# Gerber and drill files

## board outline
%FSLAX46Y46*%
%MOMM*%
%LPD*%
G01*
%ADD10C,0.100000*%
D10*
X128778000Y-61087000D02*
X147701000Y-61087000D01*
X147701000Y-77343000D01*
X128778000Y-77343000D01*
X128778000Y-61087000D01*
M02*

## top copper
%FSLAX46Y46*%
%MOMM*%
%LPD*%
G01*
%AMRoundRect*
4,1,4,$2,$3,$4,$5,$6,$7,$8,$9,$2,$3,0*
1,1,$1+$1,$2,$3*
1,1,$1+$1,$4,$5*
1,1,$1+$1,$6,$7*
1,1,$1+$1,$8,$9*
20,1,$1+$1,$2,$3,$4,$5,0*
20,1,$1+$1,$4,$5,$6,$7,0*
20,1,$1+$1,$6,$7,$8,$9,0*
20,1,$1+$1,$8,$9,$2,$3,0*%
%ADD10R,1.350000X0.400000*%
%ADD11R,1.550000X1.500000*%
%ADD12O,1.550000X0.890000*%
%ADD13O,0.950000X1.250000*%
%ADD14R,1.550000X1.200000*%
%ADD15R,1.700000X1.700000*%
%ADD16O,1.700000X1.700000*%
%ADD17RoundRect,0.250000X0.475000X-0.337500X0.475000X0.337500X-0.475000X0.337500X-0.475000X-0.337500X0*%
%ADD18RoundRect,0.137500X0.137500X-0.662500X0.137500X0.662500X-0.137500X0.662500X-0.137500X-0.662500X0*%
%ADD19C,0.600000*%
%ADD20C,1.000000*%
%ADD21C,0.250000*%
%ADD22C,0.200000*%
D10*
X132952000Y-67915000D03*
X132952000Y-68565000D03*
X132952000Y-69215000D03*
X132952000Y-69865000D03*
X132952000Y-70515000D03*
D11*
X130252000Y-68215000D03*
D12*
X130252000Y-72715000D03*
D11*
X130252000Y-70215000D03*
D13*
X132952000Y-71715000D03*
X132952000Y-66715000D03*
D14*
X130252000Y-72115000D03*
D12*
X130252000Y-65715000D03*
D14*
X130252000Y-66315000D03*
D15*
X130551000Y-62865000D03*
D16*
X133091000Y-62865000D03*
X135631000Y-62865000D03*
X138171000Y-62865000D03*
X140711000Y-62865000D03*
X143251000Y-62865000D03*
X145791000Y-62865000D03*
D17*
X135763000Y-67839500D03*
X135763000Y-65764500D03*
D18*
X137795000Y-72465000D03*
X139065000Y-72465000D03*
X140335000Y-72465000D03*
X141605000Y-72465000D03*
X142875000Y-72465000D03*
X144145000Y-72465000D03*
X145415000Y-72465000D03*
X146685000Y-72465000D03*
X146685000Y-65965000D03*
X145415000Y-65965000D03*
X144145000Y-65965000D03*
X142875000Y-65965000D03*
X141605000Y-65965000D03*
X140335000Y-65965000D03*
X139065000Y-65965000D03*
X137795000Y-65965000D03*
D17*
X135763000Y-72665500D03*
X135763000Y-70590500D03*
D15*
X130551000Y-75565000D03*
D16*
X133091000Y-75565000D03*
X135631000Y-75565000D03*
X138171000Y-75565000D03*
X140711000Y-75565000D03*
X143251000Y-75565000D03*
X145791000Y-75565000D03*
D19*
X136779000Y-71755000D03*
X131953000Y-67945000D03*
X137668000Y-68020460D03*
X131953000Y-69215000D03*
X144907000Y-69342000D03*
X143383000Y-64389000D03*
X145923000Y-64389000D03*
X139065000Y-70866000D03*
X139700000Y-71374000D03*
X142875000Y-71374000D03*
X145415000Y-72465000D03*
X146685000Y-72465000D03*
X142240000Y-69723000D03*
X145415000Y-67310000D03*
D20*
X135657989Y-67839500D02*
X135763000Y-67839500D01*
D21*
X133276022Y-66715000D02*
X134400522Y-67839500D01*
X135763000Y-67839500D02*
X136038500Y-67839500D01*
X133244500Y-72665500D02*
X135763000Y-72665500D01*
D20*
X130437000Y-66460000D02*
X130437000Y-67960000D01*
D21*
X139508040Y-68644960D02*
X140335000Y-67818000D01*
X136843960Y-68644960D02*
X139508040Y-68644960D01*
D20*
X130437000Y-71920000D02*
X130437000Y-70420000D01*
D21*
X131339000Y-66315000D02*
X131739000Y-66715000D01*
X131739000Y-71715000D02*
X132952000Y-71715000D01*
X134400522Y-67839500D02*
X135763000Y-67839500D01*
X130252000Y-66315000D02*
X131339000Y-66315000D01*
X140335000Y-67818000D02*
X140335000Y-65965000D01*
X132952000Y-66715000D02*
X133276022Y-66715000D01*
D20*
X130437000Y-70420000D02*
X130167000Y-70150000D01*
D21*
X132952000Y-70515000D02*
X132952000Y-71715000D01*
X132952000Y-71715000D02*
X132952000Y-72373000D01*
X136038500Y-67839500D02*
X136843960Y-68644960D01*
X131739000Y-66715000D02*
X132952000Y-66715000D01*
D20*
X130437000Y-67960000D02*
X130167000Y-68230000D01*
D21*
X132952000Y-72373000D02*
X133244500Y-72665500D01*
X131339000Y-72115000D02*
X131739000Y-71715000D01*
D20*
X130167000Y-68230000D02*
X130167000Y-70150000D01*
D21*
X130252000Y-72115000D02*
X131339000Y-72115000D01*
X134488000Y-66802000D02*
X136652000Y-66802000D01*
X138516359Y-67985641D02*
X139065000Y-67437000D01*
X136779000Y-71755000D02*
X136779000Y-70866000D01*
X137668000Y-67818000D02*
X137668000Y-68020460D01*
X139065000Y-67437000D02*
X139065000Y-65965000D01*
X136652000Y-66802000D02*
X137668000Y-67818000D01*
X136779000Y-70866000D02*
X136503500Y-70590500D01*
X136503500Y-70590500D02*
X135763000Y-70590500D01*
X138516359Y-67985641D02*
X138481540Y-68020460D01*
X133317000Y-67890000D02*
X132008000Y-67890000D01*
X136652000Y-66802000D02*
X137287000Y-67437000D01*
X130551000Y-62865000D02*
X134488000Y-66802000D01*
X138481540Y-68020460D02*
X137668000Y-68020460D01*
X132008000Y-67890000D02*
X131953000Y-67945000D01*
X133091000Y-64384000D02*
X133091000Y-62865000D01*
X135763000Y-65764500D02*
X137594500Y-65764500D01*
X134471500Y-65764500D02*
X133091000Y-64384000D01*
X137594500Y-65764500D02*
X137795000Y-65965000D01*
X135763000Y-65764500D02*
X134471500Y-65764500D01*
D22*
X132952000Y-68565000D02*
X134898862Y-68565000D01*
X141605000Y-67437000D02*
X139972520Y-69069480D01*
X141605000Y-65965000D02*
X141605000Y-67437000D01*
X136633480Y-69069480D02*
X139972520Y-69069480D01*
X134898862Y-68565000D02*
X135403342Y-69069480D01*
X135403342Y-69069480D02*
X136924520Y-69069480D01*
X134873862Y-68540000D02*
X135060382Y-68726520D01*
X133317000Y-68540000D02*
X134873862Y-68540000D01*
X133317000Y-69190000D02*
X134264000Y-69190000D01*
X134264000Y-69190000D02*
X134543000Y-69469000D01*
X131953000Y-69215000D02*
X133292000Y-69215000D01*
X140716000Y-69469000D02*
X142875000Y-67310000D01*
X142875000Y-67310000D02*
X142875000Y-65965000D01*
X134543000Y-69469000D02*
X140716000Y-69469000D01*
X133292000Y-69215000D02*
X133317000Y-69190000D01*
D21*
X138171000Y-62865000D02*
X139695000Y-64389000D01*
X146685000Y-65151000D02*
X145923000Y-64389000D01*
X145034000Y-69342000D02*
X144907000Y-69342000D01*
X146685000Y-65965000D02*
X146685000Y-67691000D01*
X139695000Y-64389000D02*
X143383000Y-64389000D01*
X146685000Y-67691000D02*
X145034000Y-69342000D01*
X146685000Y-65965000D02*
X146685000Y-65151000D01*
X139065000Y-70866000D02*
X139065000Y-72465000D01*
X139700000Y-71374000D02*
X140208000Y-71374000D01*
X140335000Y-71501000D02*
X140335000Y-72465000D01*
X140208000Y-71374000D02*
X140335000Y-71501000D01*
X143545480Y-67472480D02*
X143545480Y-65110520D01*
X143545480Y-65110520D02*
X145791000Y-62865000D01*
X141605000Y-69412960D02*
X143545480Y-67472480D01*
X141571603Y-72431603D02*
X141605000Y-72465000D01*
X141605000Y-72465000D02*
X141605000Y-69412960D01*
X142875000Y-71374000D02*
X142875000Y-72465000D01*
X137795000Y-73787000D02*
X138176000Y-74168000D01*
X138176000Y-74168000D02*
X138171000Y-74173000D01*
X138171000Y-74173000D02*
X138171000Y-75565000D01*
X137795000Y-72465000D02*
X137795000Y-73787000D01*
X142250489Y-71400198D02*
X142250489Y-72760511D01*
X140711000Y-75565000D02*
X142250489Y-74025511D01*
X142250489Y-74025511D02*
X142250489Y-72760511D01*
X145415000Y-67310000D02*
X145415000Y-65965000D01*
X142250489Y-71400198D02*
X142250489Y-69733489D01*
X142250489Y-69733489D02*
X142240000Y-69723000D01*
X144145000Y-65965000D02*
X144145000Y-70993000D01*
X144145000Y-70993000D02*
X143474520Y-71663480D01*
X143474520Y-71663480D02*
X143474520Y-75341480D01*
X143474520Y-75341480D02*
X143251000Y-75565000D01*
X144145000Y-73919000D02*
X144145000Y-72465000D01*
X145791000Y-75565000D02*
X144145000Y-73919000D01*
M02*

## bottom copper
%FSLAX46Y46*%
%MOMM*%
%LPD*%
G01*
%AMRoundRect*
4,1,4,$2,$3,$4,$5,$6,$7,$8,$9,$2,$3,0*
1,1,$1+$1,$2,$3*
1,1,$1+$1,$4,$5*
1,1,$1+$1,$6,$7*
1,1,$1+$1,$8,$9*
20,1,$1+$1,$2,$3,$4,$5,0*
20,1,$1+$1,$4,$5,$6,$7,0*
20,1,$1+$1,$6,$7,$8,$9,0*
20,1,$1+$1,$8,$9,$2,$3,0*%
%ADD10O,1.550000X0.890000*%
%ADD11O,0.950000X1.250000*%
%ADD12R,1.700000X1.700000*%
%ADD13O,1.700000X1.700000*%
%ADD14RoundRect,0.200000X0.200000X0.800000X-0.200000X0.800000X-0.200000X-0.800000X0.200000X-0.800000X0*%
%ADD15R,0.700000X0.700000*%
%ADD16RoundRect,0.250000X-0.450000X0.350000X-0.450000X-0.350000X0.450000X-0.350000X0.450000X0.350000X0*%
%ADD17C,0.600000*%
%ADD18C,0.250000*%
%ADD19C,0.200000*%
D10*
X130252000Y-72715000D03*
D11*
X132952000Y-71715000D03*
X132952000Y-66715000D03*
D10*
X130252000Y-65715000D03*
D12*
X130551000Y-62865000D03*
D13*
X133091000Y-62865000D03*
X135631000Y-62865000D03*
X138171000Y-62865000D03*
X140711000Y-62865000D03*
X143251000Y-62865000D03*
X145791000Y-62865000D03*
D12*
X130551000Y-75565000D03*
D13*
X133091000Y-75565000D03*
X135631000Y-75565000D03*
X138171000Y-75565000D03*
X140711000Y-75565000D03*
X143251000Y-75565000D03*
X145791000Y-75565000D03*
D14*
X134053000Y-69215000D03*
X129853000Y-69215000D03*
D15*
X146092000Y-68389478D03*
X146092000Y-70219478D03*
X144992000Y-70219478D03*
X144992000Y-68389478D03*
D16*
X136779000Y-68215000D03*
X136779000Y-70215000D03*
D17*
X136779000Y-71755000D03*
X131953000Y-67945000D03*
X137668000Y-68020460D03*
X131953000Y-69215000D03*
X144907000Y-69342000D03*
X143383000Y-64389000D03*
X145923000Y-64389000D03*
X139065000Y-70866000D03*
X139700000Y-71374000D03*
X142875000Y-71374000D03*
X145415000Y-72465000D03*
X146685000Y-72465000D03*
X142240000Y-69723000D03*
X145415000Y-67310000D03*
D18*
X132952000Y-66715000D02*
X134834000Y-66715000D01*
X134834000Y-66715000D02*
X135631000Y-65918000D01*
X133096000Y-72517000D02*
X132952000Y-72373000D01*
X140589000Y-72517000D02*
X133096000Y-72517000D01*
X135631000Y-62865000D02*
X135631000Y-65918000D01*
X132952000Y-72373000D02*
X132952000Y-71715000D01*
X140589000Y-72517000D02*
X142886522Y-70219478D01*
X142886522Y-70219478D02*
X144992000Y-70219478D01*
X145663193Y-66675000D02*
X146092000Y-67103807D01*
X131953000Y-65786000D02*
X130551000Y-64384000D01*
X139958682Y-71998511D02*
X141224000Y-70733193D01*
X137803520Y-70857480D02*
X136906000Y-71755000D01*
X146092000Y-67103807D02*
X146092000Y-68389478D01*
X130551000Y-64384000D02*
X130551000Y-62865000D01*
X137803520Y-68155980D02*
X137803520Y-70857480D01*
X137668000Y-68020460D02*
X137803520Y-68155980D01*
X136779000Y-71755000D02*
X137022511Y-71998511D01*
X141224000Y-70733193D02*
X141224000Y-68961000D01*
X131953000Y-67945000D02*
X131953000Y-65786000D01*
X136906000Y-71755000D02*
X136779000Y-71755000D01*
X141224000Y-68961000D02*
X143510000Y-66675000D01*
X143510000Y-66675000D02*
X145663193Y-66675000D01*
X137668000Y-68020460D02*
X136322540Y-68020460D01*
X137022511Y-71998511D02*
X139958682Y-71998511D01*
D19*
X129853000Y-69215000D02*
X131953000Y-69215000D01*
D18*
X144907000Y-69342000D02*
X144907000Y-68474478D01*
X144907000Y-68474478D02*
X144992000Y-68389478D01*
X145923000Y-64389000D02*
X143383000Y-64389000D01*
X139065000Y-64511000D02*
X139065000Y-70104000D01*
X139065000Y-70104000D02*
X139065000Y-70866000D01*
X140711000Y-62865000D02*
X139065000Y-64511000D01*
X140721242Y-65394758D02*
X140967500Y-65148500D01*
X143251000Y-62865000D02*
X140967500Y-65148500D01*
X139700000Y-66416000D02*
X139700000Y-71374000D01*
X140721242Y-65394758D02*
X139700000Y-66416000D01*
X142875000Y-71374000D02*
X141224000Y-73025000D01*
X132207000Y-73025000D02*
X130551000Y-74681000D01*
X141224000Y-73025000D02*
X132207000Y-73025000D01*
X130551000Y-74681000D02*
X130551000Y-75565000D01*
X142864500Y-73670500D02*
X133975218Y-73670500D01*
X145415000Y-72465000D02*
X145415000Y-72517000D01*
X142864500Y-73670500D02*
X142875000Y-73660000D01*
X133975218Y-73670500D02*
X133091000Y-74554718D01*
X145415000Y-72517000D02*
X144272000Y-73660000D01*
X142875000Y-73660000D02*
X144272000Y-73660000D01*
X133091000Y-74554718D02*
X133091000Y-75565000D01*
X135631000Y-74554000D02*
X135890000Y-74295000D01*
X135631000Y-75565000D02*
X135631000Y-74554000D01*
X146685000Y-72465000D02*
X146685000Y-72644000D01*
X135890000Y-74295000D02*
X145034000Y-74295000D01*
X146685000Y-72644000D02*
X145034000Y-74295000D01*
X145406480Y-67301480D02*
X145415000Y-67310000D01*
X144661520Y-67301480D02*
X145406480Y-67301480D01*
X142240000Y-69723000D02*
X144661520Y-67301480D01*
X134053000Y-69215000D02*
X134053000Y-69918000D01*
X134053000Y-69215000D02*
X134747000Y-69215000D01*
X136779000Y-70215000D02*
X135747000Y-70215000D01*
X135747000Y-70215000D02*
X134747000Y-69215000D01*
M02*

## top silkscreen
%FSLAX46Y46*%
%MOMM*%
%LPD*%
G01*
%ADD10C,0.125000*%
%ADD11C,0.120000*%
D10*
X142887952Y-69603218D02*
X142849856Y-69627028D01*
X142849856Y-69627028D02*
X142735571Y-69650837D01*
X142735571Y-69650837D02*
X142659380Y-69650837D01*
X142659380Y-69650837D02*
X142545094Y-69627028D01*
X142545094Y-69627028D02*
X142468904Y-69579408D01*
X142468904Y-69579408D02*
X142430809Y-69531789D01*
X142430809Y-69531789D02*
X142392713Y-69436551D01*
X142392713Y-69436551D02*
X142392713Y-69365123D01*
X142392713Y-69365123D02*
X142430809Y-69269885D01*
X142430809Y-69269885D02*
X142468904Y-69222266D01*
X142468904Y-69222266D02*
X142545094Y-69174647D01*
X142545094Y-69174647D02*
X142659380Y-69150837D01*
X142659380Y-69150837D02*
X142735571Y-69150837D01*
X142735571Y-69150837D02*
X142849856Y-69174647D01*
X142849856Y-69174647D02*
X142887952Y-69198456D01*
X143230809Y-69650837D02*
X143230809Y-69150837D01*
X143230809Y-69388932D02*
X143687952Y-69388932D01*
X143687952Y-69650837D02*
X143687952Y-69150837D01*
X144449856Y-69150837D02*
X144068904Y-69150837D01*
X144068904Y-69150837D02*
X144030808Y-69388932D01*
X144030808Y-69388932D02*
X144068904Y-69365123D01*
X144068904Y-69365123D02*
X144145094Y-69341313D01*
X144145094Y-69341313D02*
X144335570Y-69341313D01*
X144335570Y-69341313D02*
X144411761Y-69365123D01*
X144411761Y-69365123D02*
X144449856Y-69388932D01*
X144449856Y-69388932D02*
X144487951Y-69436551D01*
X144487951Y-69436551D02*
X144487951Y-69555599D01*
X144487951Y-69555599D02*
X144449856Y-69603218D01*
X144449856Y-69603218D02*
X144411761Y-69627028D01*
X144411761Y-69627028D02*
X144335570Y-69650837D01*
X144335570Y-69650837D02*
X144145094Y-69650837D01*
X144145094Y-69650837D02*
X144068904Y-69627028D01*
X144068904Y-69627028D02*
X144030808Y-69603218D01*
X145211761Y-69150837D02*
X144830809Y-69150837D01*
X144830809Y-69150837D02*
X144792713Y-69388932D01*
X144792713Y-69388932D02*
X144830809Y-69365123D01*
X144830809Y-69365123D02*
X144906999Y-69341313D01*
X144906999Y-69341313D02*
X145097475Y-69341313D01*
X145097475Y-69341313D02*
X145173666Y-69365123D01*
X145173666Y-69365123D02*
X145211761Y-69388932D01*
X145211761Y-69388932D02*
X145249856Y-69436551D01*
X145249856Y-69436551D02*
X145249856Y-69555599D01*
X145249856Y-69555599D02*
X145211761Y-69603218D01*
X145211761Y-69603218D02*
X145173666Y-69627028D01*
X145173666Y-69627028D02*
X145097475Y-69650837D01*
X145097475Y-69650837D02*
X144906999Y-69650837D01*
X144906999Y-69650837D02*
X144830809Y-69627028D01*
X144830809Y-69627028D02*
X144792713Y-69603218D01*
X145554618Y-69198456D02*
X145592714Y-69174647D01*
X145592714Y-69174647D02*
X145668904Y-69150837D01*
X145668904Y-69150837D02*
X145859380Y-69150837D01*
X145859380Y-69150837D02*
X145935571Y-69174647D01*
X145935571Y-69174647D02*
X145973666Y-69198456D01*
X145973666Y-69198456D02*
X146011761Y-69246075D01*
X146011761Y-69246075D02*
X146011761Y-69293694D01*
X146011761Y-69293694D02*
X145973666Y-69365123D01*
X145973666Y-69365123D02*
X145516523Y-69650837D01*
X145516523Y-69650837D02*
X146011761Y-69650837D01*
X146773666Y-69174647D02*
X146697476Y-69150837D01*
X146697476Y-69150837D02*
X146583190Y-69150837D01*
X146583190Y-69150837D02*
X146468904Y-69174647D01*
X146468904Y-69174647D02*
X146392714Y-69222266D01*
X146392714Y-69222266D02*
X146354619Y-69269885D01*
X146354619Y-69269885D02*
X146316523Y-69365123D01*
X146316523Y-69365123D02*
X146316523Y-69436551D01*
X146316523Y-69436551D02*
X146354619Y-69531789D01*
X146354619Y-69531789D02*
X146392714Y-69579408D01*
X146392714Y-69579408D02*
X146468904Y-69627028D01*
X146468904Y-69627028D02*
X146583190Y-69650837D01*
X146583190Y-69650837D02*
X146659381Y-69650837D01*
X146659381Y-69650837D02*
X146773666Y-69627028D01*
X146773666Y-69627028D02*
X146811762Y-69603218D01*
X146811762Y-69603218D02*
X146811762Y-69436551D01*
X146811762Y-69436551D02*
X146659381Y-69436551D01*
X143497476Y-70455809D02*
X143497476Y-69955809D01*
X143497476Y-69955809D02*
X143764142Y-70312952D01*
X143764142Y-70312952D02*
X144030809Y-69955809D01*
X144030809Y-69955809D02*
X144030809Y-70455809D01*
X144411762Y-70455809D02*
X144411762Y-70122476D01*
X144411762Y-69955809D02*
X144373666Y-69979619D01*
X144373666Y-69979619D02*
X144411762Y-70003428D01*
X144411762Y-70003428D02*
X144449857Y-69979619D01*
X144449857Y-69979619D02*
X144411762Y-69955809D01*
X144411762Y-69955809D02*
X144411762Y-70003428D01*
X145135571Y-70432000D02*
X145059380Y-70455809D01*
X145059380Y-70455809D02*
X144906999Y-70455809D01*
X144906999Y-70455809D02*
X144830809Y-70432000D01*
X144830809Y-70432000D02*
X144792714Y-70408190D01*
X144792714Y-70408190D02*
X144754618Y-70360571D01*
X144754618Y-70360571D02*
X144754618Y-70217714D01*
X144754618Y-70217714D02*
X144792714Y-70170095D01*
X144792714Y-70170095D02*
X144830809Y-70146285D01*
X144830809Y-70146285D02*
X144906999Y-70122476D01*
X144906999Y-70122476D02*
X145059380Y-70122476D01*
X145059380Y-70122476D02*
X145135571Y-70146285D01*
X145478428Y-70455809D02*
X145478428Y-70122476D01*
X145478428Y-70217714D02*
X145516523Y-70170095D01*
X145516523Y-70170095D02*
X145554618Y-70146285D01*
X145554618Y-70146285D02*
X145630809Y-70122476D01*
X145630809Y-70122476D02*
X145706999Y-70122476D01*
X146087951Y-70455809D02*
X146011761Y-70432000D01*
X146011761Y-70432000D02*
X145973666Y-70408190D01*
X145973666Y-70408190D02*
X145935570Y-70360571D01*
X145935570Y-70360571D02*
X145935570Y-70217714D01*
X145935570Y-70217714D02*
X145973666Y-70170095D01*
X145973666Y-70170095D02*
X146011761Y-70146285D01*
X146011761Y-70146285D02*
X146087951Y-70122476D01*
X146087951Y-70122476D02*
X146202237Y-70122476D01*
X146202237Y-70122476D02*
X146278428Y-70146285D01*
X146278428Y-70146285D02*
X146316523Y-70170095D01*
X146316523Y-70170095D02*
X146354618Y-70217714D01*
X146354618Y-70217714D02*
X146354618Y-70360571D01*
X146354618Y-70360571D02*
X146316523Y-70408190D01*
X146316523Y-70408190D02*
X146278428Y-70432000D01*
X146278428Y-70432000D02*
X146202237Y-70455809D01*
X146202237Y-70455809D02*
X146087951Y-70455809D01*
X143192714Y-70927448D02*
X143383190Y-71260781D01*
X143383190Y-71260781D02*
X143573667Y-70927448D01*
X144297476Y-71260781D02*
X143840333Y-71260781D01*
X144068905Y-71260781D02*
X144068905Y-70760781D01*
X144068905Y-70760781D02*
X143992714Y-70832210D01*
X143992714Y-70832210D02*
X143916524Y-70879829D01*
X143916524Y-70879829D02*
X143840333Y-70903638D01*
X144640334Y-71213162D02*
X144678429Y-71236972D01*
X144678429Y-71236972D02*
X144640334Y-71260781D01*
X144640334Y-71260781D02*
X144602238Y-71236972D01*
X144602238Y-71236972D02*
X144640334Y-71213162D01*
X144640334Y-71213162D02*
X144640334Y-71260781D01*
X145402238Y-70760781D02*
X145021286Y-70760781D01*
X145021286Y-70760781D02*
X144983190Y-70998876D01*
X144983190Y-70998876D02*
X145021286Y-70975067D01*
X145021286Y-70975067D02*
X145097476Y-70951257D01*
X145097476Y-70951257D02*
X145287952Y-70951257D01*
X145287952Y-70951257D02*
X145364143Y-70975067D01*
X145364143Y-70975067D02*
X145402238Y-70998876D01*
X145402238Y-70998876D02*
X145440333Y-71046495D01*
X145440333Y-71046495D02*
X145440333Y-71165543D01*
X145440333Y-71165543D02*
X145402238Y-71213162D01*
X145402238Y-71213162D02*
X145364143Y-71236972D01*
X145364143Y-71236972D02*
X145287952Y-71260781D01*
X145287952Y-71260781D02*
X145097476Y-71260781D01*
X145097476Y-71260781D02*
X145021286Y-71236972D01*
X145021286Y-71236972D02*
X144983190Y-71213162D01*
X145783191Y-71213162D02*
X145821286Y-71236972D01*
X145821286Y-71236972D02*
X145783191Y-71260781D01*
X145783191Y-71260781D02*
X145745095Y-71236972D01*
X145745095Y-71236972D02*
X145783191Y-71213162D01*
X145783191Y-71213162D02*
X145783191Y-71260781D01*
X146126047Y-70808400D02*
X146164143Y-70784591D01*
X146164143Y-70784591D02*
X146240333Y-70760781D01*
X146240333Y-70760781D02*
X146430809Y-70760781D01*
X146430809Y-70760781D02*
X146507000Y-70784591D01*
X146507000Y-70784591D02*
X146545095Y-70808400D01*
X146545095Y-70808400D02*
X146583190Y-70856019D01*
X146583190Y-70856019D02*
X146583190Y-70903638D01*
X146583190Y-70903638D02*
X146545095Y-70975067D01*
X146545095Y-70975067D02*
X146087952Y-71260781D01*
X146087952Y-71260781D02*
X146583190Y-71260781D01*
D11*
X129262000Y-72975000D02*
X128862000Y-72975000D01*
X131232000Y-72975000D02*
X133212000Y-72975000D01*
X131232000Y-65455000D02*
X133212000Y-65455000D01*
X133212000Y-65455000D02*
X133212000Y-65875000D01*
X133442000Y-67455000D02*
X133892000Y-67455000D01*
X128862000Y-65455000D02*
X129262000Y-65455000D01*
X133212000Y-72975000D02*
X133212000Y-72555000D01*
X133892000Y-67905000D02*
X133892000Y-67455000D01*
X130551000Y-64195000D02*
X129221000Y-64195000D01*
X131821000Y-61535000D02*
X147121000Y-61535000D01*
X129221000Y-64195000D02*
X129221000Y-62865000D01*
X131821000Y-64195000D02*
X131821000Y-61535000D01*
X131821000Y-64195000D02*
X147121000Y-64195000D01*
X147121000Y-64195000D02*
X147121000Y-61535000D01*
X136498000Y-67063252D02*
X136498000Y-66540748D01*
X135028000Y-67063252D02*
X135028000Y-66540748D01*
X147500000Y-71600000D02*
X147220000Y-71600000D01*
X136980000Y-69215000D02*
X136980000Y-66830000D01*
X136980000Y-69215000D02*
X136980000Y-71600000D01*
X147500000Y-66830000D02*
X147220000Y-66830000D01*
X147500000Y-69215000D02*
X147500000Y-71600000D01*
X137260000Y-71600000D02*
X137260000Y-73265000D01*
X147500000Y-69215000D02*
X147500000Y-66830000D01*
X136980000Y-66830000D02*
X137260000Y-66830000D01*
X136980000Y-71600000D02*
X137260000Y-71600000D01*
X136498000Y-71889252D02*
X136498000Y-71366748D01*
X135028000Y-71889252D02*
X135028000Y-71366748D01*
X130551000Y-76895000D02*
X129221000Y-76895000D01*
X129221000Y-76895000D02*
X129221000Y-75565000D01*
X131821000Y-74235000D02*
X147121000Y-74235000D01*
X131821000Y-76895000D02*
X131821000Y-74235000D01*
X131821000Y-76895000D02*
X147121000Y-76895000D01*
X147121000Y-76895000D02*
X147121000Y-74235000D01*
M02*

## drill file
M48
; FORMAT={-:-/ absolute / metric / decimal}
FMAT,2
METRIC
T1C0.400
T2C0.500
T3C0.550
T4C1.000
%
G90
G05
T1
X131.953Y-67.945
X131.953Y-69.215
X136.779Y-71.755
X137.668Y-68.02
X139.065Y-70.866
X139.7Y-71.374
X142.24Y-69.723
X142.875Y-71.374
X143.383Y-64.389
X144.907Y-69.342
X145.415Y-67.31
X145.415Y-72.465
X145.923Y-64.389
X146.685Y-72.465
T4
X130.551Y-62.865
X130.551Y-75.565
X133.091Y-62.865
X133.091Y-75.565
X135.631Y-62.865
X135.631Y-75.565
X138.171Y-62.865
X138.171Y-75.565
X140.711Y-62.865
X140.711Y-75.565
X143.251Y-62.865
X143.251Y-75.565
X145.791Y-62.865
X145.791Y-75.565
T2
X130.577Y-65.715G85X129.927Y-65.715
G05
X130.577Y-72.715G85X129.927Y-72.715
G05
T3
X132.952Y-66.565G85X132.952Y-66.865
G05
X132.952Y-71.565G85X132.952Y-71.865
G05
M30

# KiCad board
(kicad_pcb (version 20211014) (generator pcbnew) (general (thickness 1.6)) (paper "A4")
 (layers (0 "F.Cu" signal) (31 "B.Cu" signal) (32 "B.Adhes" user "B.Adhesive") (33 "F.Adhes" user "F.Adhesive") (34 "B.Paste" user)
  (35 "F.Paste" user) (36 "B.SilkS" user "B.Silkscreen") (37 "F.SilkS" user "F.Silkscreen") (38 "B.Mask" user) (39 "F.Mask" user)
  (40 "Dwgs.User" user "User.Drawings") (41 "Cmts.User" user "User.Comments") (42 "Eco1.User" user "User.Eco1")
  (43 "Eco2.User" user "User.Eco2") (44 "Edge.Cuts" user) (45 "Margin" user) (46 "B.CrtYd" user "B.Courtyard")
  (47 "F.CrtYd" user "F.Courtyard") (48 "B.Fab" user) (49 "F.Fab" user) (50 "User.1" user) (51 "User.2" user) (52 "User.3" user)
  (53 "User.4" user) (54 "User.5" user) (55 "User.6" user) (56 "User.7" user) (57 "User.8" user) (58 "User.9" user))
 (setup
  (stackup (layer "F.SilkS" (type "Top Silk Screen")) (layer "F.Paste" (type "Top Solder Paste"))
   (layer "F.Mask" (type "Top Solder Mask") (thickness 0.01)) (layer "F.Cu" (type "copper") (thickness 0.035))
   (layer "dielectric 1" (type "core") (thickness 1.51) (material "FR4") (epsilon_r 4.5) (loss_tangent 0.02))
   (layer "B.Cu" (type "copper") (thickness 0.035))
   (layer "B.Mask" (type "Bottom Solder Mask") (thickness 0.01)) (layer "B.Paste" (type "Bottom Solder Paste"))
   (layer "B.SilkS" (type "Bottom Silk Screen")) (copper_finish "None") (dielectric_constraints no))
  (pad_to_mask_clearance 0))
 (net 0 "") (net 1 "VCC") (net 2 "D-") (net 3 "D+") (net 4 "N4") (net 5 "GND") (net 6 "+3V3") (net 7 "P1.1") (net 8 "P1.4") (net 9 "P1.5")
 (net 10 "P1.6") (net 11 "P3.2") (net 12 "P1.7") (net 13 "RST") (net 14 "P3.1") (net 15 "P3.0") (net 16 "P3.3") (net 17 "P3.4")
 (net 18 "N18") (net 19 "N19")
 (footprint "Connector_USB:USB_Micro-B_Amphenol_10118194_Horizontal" (layer "F.Cu") (at 131.552 69.215 -90)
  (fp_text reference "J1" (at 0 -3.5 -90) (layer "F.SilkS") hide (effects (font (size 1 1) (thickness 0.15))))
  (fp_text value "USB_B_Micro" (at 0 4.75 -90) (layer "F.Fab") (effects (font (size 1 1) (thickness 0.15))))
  (fp_line (start 3.76 2.29) (end 3.76 2.69) (layer "F.SilkS") (width 0.12))
  (fp_line (start 3.76 0.32) (end 3.76 -1.66) (layer "F.SilkS") (width 0.12))
  (fp_line (start -3.76 0.32) (end -3.76 -1.66) (layer "F.SilkS") (width 0.12))
  (fp_line (start -3.76 -1.66) (end -3.34 -1.66) (layer "F.SilkS") (width 0.12))
  (fp_line (start -1.76 -1.89) (end -1.76 -2.34) (layer "F.SilkS") (width 0.12))
  (fp_line (start -3.76 2.69) (end -3.76 2.29) (layer "F.SilkS") (width 0.12))
  (fp_line (start 3.76 -1.66) (end 3.34 -1.66) (layer "F.SilkS") (width 0.12))
  (fp_line (start -1.31 -2.34) (end -1.76 -2.34) (layer "F.SilkS") (width 0.12))
  (pad "" smd oval (at -3.5 1.3 270) (size 0.89 1.55) (layers "F.Paste"))
  (pad "" smd oval (at 2.5 -1.4 270) (size 1.25 0.95) (layers "F.Paste"))
  (pad "" smd oval (at 3.5 1.3 270) (size 0.89 1.55) (layers "F.Paste"))
  (pad "" smd oval (at -2.5 -1.4 270) (size 1.25 0.95) (layers "F.Paste"))
  (pad "1" smd rect (at -1.3 -1.4 270) (size 0.4 1.35) (layers "F.Cu" "F.Paste" "F.Mask") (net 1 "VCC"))
  (pad "2" smd rect (at -0.65 -1.4 270) (size 0.4 1.35) (layers "F.Cu" "F.Paste" "F.Mask") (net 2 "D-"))
  (pad "3" smd rect (at 0 -1.4 270) (size 0.4 1.35) (layers "F.Cu" "F.Paste" "F.Mask") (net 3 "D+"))
  (pad "4" smd rect (at 0.65 -1.4 270) (size 0.4 1.35) (layers "F.Cu" "F.Paste" "F.Mask") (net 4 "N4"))
  (pad "5" smd rect (at 1.3 -1.4 270) (size 0.4 1.35) (layers "F.Cu" "F.Paste" "F.Mask") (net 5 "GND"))
  (pad "6" smd rect (at -1 1.3 270) (size 1.5 1.55) (layers "F.Cu" "F.Paste" "F.Mask") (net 5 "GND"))
  (pad "6" thru_hole oval (at 3.5 1.3 270) (size 0.89 1.55) (drill oval 0.5 1.15) (layers *.Cu *.Mask) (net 5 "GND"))
  (pad "6" smd rect (at 1 1.3 270) (size 1.5 1.55) (layers "F.Cu" "F.Paste" "F.Mask") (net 5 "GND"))
  (pad "6" thru_hole oval (at 2.5 -1.4 270) (size 1.25 0.95) (drill oval 0.85 0.55) (layers *.Cu *.Mask) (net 5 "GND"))
  (pad "6" thru_hole oval (at -2.5 -1.4 270) (size 1.25 0.95) (drill oval 0.85 0.55) (layers *.Cu *.Mask) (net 5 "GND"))
  (pad "6" smd rect (at 2.9 1.3 270) (size 1.2 1.55) (layers "F.Cu" "F.Paste" "F.Mask") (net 5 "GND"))
  (pad "6" thru_hole oval (at -3.5 1.3 270) (size 0.89 1.55) (drill oval 0.5 1.15) (layers *.Cu *.Mask) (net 5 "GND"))
  (pad "6" smd rect (at -2.9 1.3 270) (size 1.2 1.55) (layers "F.Cu" "F.Paste" "F.Mask") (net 5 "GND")))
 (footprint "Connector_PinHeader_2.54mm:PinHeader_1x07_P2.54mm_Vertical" (layer "F.Cu") (at 130.551 62.865 90)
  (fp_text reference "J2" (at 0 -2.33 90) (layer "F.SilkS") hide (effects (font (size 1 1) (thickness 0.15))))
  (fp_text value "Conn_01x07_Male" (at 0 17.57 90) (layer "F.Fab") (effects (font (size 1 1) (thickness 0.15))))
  (fp_line (start -1.33 0) (end -1.33 -1.33) (layer "F.SilkS") (width 0.12))
  (fp_line (start 1.33 1.27) (end 1.33 16.57) (layer "F.SilkS") (width 0.12))
  (fp_line (start -1.33 -1.33) (end 0 -1.33) (layer "F.SilkS") (width 0.12))
  (fp_line (start -1.33 1.27) (end 1.33 1.27) (layer "F.SilkS") (width 0.12))
  (fp_line (start -1.33 1.27) (end -1.33 16.57) (layer "F.SilkS") (width 0.12))
  (fp_line (start -1.33 16.57) (end 1.33 16.57) (layer "F.SilkS") (width 0.12))
  (pad "1" thru_hole rect (at 0 0 90) (size 1.7 1.7) (drill 1) (layers *.Cu *.Mask) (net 1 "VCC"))
  (pad "2" thru_hole oval (at 0 2.54 90) (size 1.7 1.7) (drill 1) (layers *.Cu *.Mask) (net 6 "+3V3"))
  (pad "3" thru_hole oval (at 0 5.08 90) (size 1.7 1.7) (drill 1) (layers *.Cu *.Mask) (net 5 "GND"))
  (pad "4" thru_hole oval (at 0 7.62 90) (size 1.7 1.7) (drill 1) (layers *.Cu *.Mask) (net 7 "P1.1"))
  (pad "5" thru_hole oval (at 0 10.16 90) (size 1.7 1.7) (drill 1) (layers *.Cu *.Mask) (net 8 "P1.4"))
  (pad "6" thru_hole oval (at 0 12.7 90) (size 1.7 1.7) (drill 1) (layers *.Cu *.Mask) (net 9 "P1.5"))
  (pad "7" thru_hole oval (at 0 15.24 90) (size 1.7 1.7) (drill 1) (layers *.Cu *.Mask) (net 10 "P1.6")))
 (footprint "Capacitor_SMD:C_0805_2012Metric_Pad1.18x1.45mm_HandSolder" (layer "F.Cu") (at 135.763 66.802 90)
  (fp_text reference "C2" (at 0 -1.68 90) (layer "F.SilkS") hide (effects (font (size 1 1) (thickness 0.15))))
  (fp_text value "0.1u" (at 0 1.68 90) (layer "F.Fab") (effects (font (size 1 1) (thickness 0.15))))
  (fp_line (start -0.261252 0.735) (end 0.261252 0.735) (layer "F.SilkS") (width 0.12))
  (fp_line (start -0.261252 -0.735) (end 0.261252 -0.735) (layer "F.SilkS") (width 0.12))
  (pad "1" smd roundrect (at -1.0375 0 90) (size 1.175 1.45) (layers "F.Cu" "F.Paste" "F.Mask") (roundrect_rratio 0.2127659574)
   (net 5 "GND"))
  (pad "2" smd roundrect (at 1.0375 0 90) (size 1.175 1.45) (layers "F.Cu" "F.Paste" "F.Mask") (roundrect_rratio 0.2127659574)
   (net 6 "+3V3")))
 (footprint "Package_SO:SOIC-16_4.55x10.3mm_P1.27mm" (layer "F.Cu") (at 142.24 69.215 90)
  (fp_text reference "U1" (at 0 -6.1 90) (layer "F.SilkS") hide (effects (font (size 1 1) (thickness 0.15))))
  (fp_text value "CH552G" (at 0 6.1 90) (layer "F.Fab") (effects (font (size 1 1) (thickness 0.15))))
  (fp_line (start -2.385 5.26) (end -2.385 4.98) (layer "F.SilkS") (width 0.12))
  (fp_line (start 0 -5.26) (end 2.385 -5.26) (layer "F.SilkS") (width 0.12))
  (fp_line (start 0 -5.26) (end -2.385 -5.26) (layer "F.SilkS") (width 0.12))
  (fp_line (start 2.385 5.26) (end 2.385 4.98) (layer "F.SilkS") (width 0.12))
  (fp_line (start 0 5.26) (end -2.385 5.26) (layer "F.SilkS") (width 0.12))
  (fp_line (start -2.385 -4.98) (end -4.05 -4.98) (layer "F.SilkS") (width 0.12))
  (fp_line (start 0 5.26) (end 2.385 5.26) (layer "F.SilkS") (width 0.12))
  (fp_line (start 2.385 -5.26) (end 2.385 -4.98) (layer "F.SilkS") (width 0.12))
  (fp_line (start -2.385 -5.26) (end -2.385 -4.98) (layer "F.SilkS") (width 0.12))
  (pad "1" smd roundrect (at -3.25 -4.445 90) (size 1.6 0.55) (layers "F.Cu" "F.Paste" "F.Mask") (roundrect_rratio 0.25) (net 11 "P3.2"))
  (pad "2" smd roundrect (at -3.25 -3.175 90) (size 1.6 0.55) (layers "F.Cu" "F.Paste" "F.Mask") (roundrect_rratio 0.25) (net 8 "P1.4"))
  (pad "3" smd roundrect (at -3.25 -1.905 90) (size 1.6 0.55) (layers "F.Cu" "F.Paste" "F.Mask") (roundrect_rratio 0.25) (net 9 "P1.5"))
  (pad "4" smd roundrect (at -3.25 -0.635 90) (size 1.6 0.55) (layers "F.Cu" "F.Paste" "F.Mask") (roundrect_rratio 0.25) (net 10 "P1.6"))
  (pad "5" smd roundrect (at -3.25 0.635 90) (size 1.6 0.55) (layers "F.Cu" "F.Paste" "F.Mask") (roundrect_rratio 0.25) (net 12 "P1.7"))
  (pad "6" smd roundrect (at -3.25 1.905 90) (size 1.6 0.55) (layers "F.Cu" "F.Paste" "F.Mask") (roundrect_rratio 0.25) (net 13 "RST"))
  (pad "7" smd roundrect (at -3.25 3.175 90) (size 1.6 0.55) (layers "F.Cu" "F.Paste" "F.Mask") (roundrect_rratio 0.25) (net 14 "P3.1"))
  (pad "8" smd roundrect (at -3.25 4.445 90) (size 1.6 0.55) (layers "F.Cu" "F.Paste" "F.Mask") (roundrect_rratio 0.25) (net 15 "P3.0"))
  (pad "9" smd roundrect (at 3.25 4.445 90) (size 1.6 0.55) (layers "F.Cu" "F.Paste" "F.Mask") (roundrect_rratio 0.25) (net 7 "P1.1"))
  (pad "10" smd roundrect (at 3.25 3.175 90) (size 1.6 0.55) (layers "F.Cu" "F.Paste" "F.Mask") (roundrect_rratio 0.25) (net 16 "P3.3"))
  (pad "11" smd roundrect (at 3.25 1.905 90) (size 1.6 0.55) (layers "F.Cu" "F.Paste" "F.Mask") (roundrect_rratio 0.25) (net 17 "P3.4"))
  (pad "12" smd roundrect (at 3.25 0.635 90) (size 1.6 0.55) (layers "F.Cu" "F.Paste" "F.Mask") (roundrect_rratio 0.25) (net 3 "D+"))
  (pad "13" smd roundrect (at 3.25 -0.635 90) (size 1.6 0.55) (layers "F.Cu" "F.Paste" "F.Mask") (roundrect_rratio 0.25) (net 2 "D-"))
  (pad "14" smd roundrect (at 3.25 -1.905 90) (size 1.6 0.55) (layers "F.Cu" "F.Paste" "F.Mask") (roundrect_rratio 0.25) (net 5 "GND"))
  (pad "15" smd roundrect (at 3.25 -3.175 90) (size 1.6 0.55) (layers "F.Cu" "F.Paste" "F.Mask") (roundrect_rratio 0.25) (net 1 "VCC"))
  (pad "16" smd roundrect (at 3.25 -4.445 90) (size 1.6 0.55) (layers "F.Cu" "F.Paste" "F.Mask") (roundrect_rratio 0.25) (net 6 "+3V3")))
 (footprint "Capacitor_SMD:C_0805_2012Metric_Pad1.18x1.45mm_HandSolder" (layer "F.Cu") (at 135.763 71.628 90)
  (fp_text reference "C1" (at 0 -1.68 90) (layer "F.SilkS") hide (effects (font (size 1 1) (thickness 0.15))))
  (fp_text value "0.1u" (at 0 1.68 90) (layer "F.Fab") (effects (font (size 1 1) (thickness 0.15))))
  (fp_line (start -0.261252 0.735) (end 0.261252 0.735) (layer "F.SilkS") (width 0.12))
  (fp_line (start -0.261252 -0.735) (end 0.261252 -0.735) (layer "F.SilkS") (width 0.12))
  (pad "1" smd roundrect (at -1.0375 0 90) (size 1.175 1.45) (layers "F.Cu" "F.Paste" "F.Mask") (roundrect_rratio 0.2127659574)
   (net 5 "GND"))
  (pad "2" smd roundrect (at 1.0375 0 90) (size 1.175 1.45) (layers "F.Cu" "F.Paste" "F.Mask") (roundrect_rratio 0.2127659574) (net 1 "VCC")))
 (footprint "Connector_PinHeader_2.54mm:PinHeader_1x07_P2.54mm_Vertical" (layer "F.Cu") (at 130.551 75.565 90)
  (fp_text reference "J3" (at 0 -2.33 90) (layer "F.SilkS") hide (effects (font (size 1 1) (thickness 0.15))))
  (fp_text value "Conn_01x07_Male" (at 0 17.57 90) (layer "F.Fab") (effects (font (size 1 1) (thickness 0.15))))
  (fp_line (start -1.33 0) (end -1.33 -1.33) (layer "F.SilkS") (width 0.12))
  (fp_line (start -1.33 -1.33) (end 0 -1.33) (layer "F.SilkS") (width 0.12))
  (fp_line (start 1.33 1.27) (end 1.33 16.57) (layer "F.SilkS") (width 0.12))
  (fp_line (start -1.33 1.27) (end 1.33 1.27) (layer "F.SilkS") (width 0.12))
  (fp_line (start -1.33 1.27) (end -1.33 16.57) (layer "F.SilkS") (width 0.12))
  (fp_line (start -1.33 16.57) (end 1.33 16.57) (layer "F.SilkS") (width 0.12))
  (pad "1" thru_hole rect (at 0 0 90) (size 1.7 1.7) (drill 1) (layers *.Cu *.Mask) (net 12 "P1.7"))
  (pad "2" thru_hole oval (at 0 2.54 90) (size 1.7 1.7) (drill 1) (layers *.Cu *.Mask) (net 14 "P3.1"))
  (pad "3" thru_hole oval (at 0 5.08 90) (size 1.7 1.7) (drill 1) (layers *.Cu *.Mask) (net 15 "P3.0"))
  (pad "4" thru_hole oval (at 0 7.62 90) (size 1.7 1.7) (drill 1) (layers *.Cu *.Mask) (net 11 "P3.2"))
  (pad "5" thru_hole oval (at 0 10.16 90) (size 1.7 1.7) (drill 1) (layers *.Cu *.Mask) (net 16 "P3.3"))
  (pad "6" thru_hole oval (at 0 12.7 90) (size 1.7 1.7) (drill 1) (layers *.Cu *.Mask) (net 17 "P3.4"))
  (pad "7" thru_hole oval (at 0 15.24 90) (size 1.7 1.7) (drill 1) (layers *.Cu *.Mask) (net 13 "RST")))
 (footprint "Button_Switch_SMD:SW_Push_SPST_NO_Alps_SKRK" (layer "B.Cu") (at 131.953 69.215 180)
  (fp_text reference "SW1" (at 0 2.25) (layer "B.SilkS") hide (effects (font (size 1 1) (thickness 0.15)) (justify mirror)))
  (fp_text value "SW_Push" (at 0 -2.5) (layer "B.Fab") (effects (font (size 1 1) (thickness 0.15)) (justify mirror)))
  (pad "1" smd roundrect (at -2.1 0 180) (size 0.8 2) (layers "B.Cu" "B.Paste" "B.Mask") (roundrect_rratio 0.25) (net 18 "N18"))
  (pad "2" smd roundrect (at 2.1 0 180) (size 0.8 2) (layers "B.Cu" "B.Paste" "B.Mask") (roundrect_rratio 0.25) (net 3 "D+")))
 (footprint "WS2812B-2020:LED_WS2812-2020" (layer "B.Cu") (at 145.542 69.304478 -90)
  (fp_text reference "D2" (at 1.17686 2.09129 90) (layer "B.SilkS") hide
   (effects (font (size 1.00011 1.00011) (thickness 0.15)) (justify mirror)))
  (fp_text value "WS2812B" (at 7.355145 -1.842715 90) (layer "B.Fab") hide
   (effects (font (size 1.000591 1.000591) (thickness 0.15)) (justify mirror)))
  (pad "1" smd rect (at -0.915 -0.55 270) (size 0.7 0.7) (layers "B.Cu" "B.Paste" "B.Mask") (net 1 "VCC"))
  (pad "2" smd rect (at 0.915 -0.55 90) (size 0.7 0.7) (layers "B.Cu" "B.Paste" "B.Mask") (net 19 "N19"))
  (pad "3" smd rect (at 0.915 0.55 90) (size 0.7 0.7) (layers "B.Cu" "B.Paste" "B.Mask") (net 5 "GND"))
  (pad "4" smd rect (at -0.915 0.55 270) (size 0.7 0.7) (layers "B.Cu" "B.Paste" "B.Mask") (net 7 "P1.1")))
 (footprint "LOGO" (layer "B.Cu") (at 140.335 69.469 -45)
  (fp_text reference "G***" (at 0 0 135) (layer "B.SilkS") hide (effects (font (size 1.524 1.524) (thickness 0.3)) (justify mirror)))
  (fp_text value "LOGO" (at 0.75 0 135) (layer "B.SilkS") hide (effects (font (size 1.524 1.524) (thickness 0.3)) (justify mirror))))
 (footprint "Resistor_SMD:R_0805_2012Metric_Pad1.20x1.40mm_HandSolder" (layer "B.Cu") (at 136.779 69.215 -90)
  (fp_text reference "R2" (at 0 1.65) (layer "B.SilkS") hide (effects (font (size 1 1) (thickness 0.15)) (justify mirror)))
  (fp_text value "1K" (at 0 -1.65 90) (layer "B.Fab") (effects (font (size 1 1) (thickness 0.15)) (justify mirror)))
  (pad "1" smd roundrect (at -1 0 270) (size 1.2 1.4) (layers "B.Cu" "B.Paste" "B.Mask") (roundrect_rratio 0.208333) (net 1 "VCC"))
  (pad "2" smd roundrect (at 1 0 270) (size 1.2 1.4) (layers "B.Cu" "B.Paste" "B.Mask") (roundrect_rratio 0.208333) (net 18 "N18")))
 (gr_rect (start 147.701 77.343) (end 128.778 61.087) (layer "Edge.Cuts") (width 0.1) (fill none))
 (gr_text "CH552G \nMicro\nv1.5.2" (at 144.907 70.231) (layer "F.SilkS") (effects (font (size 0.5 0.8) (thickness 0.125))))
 (segment (start 135.657989 67.8395) (end 135.763 67.8395) (width 1) (layer "F.Cu") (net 5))
 (segment (start 133.276022 66.715) (end 134.400522 67.8395) (width 0.25) (layer "F.Cu") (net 5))
 (segment (start 135.763 67.8395) (end 136.0385 67.8395) (width 0.25) (layer "F.Cu") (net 5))
 (segment (start 133.2445 72.6655) (end 135.763 72.6655) (width 0.25) (layer "F.Cu") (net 5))
 (segment (start 130.437 66.46) (end 130.437 67.96) (width 1) (layer "F.Cu") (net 5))
 (segment (start 139.50804 68.64496) (end 140.335 67.818) (width 0.25) (layer "F.Cu") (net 5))
 (segment (start 136.84396 68.64496) (end 139.50804 68.64496) (width 0.25) (layer "F.Cu") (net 5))
 (segment (start 130.437 71.92) (end 130.437 70.42) (width 1) (layer "F.Cu") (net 5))
 (segment (start 131.339 66.315) (end 131.739 66.715) (width 0.25) (layer "F.Cu") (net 5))
 (segment (start 131.739 71.715) (end 132.952 71.715) (width 0.25) (layer "F.Cu") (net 5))
 (segment (start 134.400522 67.8395) (end 135.763 67.8395) (width 0.25) (layer "F.Cu") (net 5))
 (segment (start 130.252 66.315) (end 131.339 66.315) (width 0.25) (layer "F.Cu") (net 5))
 (segment (start 140.335 67.818) (end 140.335 65.965) (width 0.25) (layer "F.Cu") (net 5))
 (segment (start 132.952 66.715) (end 133.276022 66.715) (width 0.25) (layer "F.Cu") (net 5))
 (segment (start 130.437 70.42) (end 130.167 70.15) (width 1) (layer "F.Cu") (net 5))
 (segment (start 132.952 70.515) (end 132.952 71.715) (width 0.25) (layer "F.Cu") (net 5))
 (segment (start 132.952 71.715) (end 132.952 72.373) (width 0.25) (layer "F.Cu") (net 5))
 (segment (start 136.0385 67.8395) (end 136.84396 68.64496) (width 0.25) (layer "F.Cu") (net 5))
 (segment (start 131.739 66.715) (end 132.952 66.715) (width 0.25) (layer "F.Cu") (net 5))
 (segment (start 130.437 67.96) (end 130.167 68.23) (width 1) (layer "F.Cu") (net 5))
 (segment (start 132.952 72.373) (end 133.2445 72.6655) (width 0.25) (layer "F.Cu") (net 5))
 (segment (start 131.339 72.115) (end 131.739 71.715) (width 0.25) (layer "F.Cu") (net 5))
 (segment (start 130.167 68.23) (end 130.167 70.15) (width 1) (layer "F.Cu") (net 5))
 (segment (start 130.252 72.115) (end 131.339 72.115) (width 0.25) (layer "F.Cu") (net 5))
 (segment (start 132.952 66.715) (end 134.834 66.715) (width 0.25) (layer "B.Cu") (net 5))
 (segment (start 134.834 66.715) (end 135.631 65.918) (width 0.25) (layer "B.Cu") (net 5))
 (segment (start 133.096 72.517) (end 132.952 72.373) (width 0.25) (layer "B.Cu") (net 5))
 (segment (start 140.589 72.517) (end 133.096 72.517) (width 0.25) (layer "B.Cu") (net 5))
 (segment (start 135.631 62.865) (end 135.631 65.918) (width 0.25) (layer "B.Cu") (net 5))
 (segment (start 132.952 72.373) (end 132.952 71.715) (width 0.25) (layer "B.Cu") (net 5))
 (segment (start 140.589 72.517) (end 142.886522 70.219478) (width 0.25) (layer "B.Cu") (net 5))
 (segment (start 142.886522 70.219478) (end 144.992 70.219478) (width 0.25) (layer "B.Cu") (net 5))
 (segment (start 134.488 66.802) (end 136.652 66.802) (width 0.25) (layer "F.Cu") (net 1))
 (segment (start 138.516359 67.985641) (end 139.065 67.437) (width 0.25) (layer "F.Cu") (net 1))
 (segment (start 136.779 71.755) (end 136.779 70.866) (width 0.25) (layer "F.Cu") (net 1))
 (segment (start 137.668 67.818) (end 137.668 68.02046) (width 0.25) (layer "F.Cu") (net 1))
 (segment (start 139.065 67.437) (end 139.065 65.965) (width 0.25) (layer "F.Cu") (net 1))
 (segment (start 136.652 66.802) (end 137.668 67.818) (width 0.25) (layer "F.Cu") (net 1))
 (segment (start 136.779 70.866) (end 136.5035 70.5905) (width 0.25) (layer "F.Cu") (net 1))
 (segment (start 136.5035 70.5905) (end 135.763 70.5905) (width 0.25) (layer "F.Cu") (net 1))
 (segment (start 138.516359 67.985641) (end 138.48154 68.02046) (width 0.25) (layer "F.Cu") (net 1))
 (segment (start 133.317 67.89) (end 132.008 67.89) (width 0.25) (layer "F.Cu") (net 1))
 (segment (start 136.652 66.802) (end 137.287 67.437) (width 0.25) (layer "F.Cu") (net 1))
 (segment (start 130.551 62.865) (end 134.488 66.802) (width 0.25) (layer "F.Cu") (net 1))
 (segment (start 138.48154 68.02046) (end 137.668 68.02046) (width 0.25) (layer "F.Cu") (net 1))
 (segment (start 132.008 67.89) (end 131.953 67.945) (width 0.25) (layer "F.Cu") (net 1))
 (via (at 136.779 71.755) (size 0.6) (drill 0.4) (layers "F.Cu" "B.Cu") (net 1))
 (via (at 131.953 67.945) (size 0.6) (drill 0.4) (layers "F.Cu" "B.Cu") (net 1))
 (via (at 137.668 68.02046) (size 0.6) (drill 0.4) (layers "F.Cu" "B.Cu") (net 1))
 (segment (start 145.663193 66.675) (end 146.092 67.103807) (width 0.25) (layer "B.Cu") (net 1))
 (segment (start 131.953 65.786) (end 130.551 64.384) (width 0.25) (layer "B.Cu") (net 1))
 (segment (start 139.958682 71.998511) (end 141.224 70.733193) (width 0.25) (layer "B.Cu") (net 1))
 (segment (start 137.80352 70.85748) (end 136.906 71.755) (width 0.25) (layer "B.Cu") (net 1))
 (segment (start 146.092 67.103807) (end 146.092 68.389478) (width 0.25) (layer "B.Cu") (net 1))
 (segment (start 130.551 64.384) (end 130.551 62.865) (width 0.25) (layer "B.Cu") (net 1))
 (segment (start 137.80352 68.15598) (end 137.80352 70.85748) (width 0.25) (layer "B.Cu") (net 1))
 (segment (start 137.668 68.02046) (end 137.80352 68.15598) (width 0.25) (layer "B.Cu") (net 1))
 (segment (start 136.779 71.755) (end 137.022511 71.998511) (width 0.25) (layer "B.Cu") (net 1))
 (segment (start 141.224 70.733193) (end 141.224 68.961) (width 0.25) (layer "B.Cu") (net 1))
 (segment (start 131.953 67.945) (end 131.953 65.786) (width 0.25) (layer "B.Cu") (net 1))
 (segment (start 136.906 71.755) (end 136.779 71.755) (width 0.25) (layer "B.Cu") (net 1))
 (segment (start 141.224 68.961) (end 143.51 66.675) (width 0.25) (layer "B.Cu") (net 1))
 (segment (start 143.51 66.675) (end 145.663193 66.675) (width 0.25) (layer "B.Cu") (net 1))
 (segment (start 137.668 68.02046) (end 136.32254 68.02046) (width 0.25) (layer "B.Cu") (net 1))
 (segment (start 137.022511 71.998511) (end 139.958682 71.998511) (width 0.25) (layer "B.Cu") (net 1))
 (segment (start 133.091 64.384) (end 133.091 62.865) (width 0.25) (layer "F.Cu") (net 6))
 (segment (start 135.763 65.7645) (end 137.5945 65.7645) (width 0.25) (layer "F.Cu") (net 6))
 (segment (start 134.4715 65.7645) (end 133.091 64.384) (width 0.25) (layer "F.Cu") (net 6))
 (segment (start 137.5945 65.7645) (end 137.795 65.965) (width 0.25) (layer "F.Cu") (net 6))
 (segment (start 135.763 65.7645) (end 134.4715 65.7645) (width 0.25) (layer "F.Cu") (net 6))
 (segment (start 132.952 68.565) (end 134.898862 68.565) (width 0.2) (layer "F.Cu") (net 2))
 (segment (start 141.605 67.437) (end 139.97252 69.06948) (width 0.2) (layer "F.Cu") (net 2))
 (segment (start 141.605 65.965) (end 141.605 67.437) (width 0.2) (layer "F.Cu") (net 2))
 (segment (start 136.63348 69.06948) (end 139.97252 69.06948) (width 0.2) (layer "F.Cu") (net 2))
 (segment (start 134.898862 68.565) (end 135.403342 69.06948) (width 0.2) (layer "F.Cu") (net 2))
 (segment (start 135.403342 69.06948) (end 136.92452 69.06948) (width 0.2) (layer "F.Cu") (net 2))
 (segment (start 134.873862 68.54) (end 135.060382 68.72652) (width 0.2) (layer "F.Cu") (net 2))
 (segment (start 133.317 68.54) (end 134.873862 68.54) (width 0.2) (layer "F.Cu") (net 2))
 (segment (start 133.317 69.19) (end 134.264 69.19) (width 0.2) (layer "F.Cu") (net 3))
 (segment (start 134.264 69.19) (end 134.543 69.469) (width 0.2) (layer "F.Cu") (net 3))
 (segment (start 131.953 69.215) (end 133.292 69.215) (width 0.2) (layer "F.Cu") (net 3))
 (segment (start 140.716 69.469) (end 142.875 67.31) (width 0.2) (layer "F.Cu") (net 3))
 (segment (start 142.875 67.31) (end 142.875 65.965) (width 0.2) (layer "F.Cu") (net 3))
 (segment (start 134.543 69.469) (end 140.716 69.469) (width 0.2) (layer "F.Cu") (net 3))
 (segment (start 133.292 69.215) (end 133.317 69.19) (width 0.2) (layer "F.Cu") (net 3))
 (via (at 131.953 69.215) (size 0.6) (drill 0.4) (layers "F.Cu" "B.Cu") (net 3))
 (segment (start 129.853 69.215) (end 131.953 69.215) (width 0.2) (layer "B.Cu") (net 3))
 (segment (start 138.171 62.865) (end 139.695 64.389) (width 0.25) (layer "F.Cu") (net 7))
 (segment (start 146.685 65.151) (end 145.923 64.389) (width 0.25) (layer "F.Cu") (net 7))
 (segment (start 145.034 69.342) (end 144.907 69.342) (width 0.25) (layer "F.Cu") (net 7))
 (segment (start 146.685 65.965) (end 146.685 67.691) (width 0.25) (layer "F.Cu") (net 7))
 (segment (start 139.695 64.389) (end 143.383 64.389) (width 0.25) (layer "F.Cu") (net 7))
 (segment (start 146.685 67.691) (end 145.034 69.342) (width 0.25) (layer "F.Cu") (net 7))
 (segment (start 146.685 65.965) (end 146.685 65.151) (width 0.25) (layer "F.Cu") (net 7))
 (via (at 144.907 69.342) (size 0.6) (drill 0.4) (layers "F.Cu" "B.Cu") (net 7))
 (via (at 143.383 64.389) (size 0.6) (drill 0.4) (layers "F.Cu" "B.Cu") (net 7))
 (via (at 145.923 64.389) (size 0.6) (drill 0.4) (layers "F.Cu" "B.Cu") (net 7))
 (segment (start 144.907 69.342) (end 144.907 68.474478) (width 0.25) (layer "B.Cu") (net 7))
 (segment (start 144.907 68.474478) (end 144.992 68.389478) (width 0.25) (layer "B.Cu") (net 7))
 (segment (start 145.923 64.389) (end 143.383 64.389) (width 0.25) (layer "B.Cu") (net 7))
 (segment (start 139.065 70.866) (end 139.065 72.465) (width 0.25) (layer "F.Cu") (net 8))
 (via (at 139.065 70.866) (size 0.6) (drill 0.4) (layers "F.Cu" "B.Cu") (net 8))
 (segment (start 139.065 64.511) (end 139.065 70.104) (width 0.25) (layer "B.Cu") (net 8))
 (segment (start 139.065 70.104) (end 139.065 70.866) (width 0.25) (layer "B.Cu") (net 8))
 (segment (start 140.711 62.865) (end 139.065 64.511) (width 0.25) (layer "B.Cu") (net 8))
 (segment (start 139.7 71.374) (end 140.208 71.374) (width 0.25) (layer "F.Cu") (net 9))
 (segment (start 140.335 71.501) (end 140.335 72.465) (width 0.25) (layer "F.Cu") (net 9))
 (segment (start 140.208 71.374) (end 140.335 71.501) (width 0.25) (layer "F.Cu") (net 9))
 (via (at 139.7 71.374) (size 0.6) (drill 0.4) (layers "F.Cu" "B.Cu") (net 9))
 (segment (start 140.721242 65.394758) (end 140.9675 65.1485) (width 0.25) (layer "B.Cu") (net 9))
 (segment (start 143.251 62.865) (end 140.9675 65.1485) (width 0.25) (layer "B.Cu") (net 9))
 (segment (start 139.7 66.416) (end 139.7 71.374) (width 0.25) (layer "B.Cu") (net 9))
 (segment (start 140.721242 65.394758) (end 139.7 66.416) (width 0.25) (layer "B.Cu") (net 9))
 (segment (start 143.54548 67.47248) (end 143.54548 65.11052) (width 0.25) (layer "F.Cu") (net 10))
 (segment (start 143.54548 65.11052) (end 145.791 62.865) (width 0.25) (layer "F.Cu") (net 10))
 (segment (start 141.605 69.41296) (end 143.54548 67.47248) (width 0.25) (layer "F.Cu") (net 10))
 (segment (start 141.571603 72.431603) (end 141.605 72.465) (width 0.25) (layer "F.Cu") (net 10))
 (segment (start 141.605 72.465) (end 141.605 69.41296) (width 0.25) (layer "F.Cu") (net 10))
 (segment (start 142.875 71.374) (end 142.875 72.465) (width 0.25) (layer "F.Cu") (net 12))
 (via (at 142.875 71.374) (size 0.6) (drill 0.4) (layers "F.Cu" "B.Cu") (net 12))
 (segment (start 142.875 71.374) (end 141.224 73.025) (width 0.25) (layer "B.Cu") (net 12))
 (segment (start 132.207 73.025) (end 130.551 74.681) (width 0.25) (layer "B.Cu") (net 12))
 (segment (start 141.224 73.025) (end 132.207 73.025) (width 0.25) (layer "B.Cu") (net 12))
 (segment (start 130.551 74.681) (end 130.551 75.565) (width 0.25) (layer "B.Cu") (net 12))
 (via (at 145.415 72.465) (size 0.6) (drill 0.4) (layers "F.Cu" "B.Cu") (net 14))
 (segment (start 142.8645 73.6705) (end 133.975218 73.6705) (width 0.25) (layer "B.Cu") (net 14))
 (segment (start 145.415 72.465) (end 145.415 72.517) (width 0.25) (layer "B.Cu") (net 14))
 (segment (start 142.8645 73.6705) (end 142.875 73.66) (width 0.25) (layer "B.Cu") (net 14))
 (segment (start 133.975218 73.6705) (end 133.091 74.554718) (width 0.25) (layer "B.Cu") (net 14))
 (segment (start 145.415 72.517) (end 144.272 73.66) (width 0.25) (layer "B.Cu") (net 14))
 (segment (start 142.875 73.66) (end 144.272 73.66) (width 0.25) (layer "B.Cu") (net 14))
 (segment (start 133.091 74.554718) (end 133.091 75.565) (width 0.25) (layer "B.Cu") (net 14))
 (via (at 146.685 72.465) (size 0.6) (drill 0.4) (layers "F.Cu" "B.Cu") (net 15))
 (segment (start 135.631 74.554) (end 135.89 74.295) (width 0.25) (layer "B.Cu") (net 15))
 (segment (start 135.631 75.565) (end 135.631 74.554) (width 0.25) (layer "B.Cu") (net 15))
 (segment (start 146.685 72.465) (end 146.685 72.644) (width 0.25) (layer "B.Cu") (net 15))
 (segment (start 135.89 74.295) (end 145.034 74.295) (width 0.25) (layer "B.Cu") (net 15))
 (segment (start 146.685 72.644) (end 145.034 74.295) (width 0.25) (layer "B.Cu") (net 15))
 (segment (start 137.795 73.787) (end 138.176 74.168) (width 0.25) (layer "F.Cu") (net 11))
 (segment (start 138.176 74.168) (end 138.171 74.173) (width 0.25) (layer "F.Cu") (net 11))
 (segment (start 138.171 74.173) (end 138.171 75.565) (width 0.25) (layer "F.Cu") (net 11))
 (segment (start 137.795 72.465) (end 137.795 73.787) (width 0.25) (layer "F.Cu") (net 11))
 (segment (start 142.250489 71.400198) (end 142.250489 72.760511) (width 0.25) (layer "F.Cu") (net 16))
 (segment (start 140.711 75.565) (end 142.250489 74.025511) (width 0.25) (layer "F.Cu") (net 16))
 (segment (start 142.250489 74.025511) (end 142.250489 72.760511) (width 0.25) (layer "F.Cu") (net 16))
 (segment (start 145.415 67.31) (end 145.415 65.965) (width 0.25) (layer "F.Cu") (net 16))
 (segment (start 142.250489 71.400198) (end 142.250489 69.733489) (width 0.25) (layer "F.Cu") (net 16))
 (segment (start 142.250489 69.733489) (end 142.24 69.723) (width 0.25) (layer "F.Cu") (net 16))
 (via (at 142.24 69.723) (size 0.6) (drill 0.4) (layers "F.Cu" "B.Cu") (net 16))
 (via (at 145.415 67.31) (size 0.6) (drill 0.4) (layers "F.Cu" "B.Cu") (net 16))
 (segment (start 145.40648 67.30148) (end 145.415 67.31) (width 0.25) (layer "B.Cu") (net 16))
 (segment (start 144.66152 67.30148) (end 145.40648 67.30148) (width 0.25) (layer "B.Cu") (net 16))
 (segment (start 142.24 69.723) (end 144.66152 67.30148) (width 0.25) (layer "B.Cu") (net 16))
 (segment (start 144.145 65.965) (end 144.145 70.993) (width 0.25) (layer "F.Cu") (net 17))
 (segment (start 144.145 70.993) (end 143.47452 71.66348) (width 0.25) (layer "F.Cu") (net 17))
 (segment (start 143.47452 71.66348) (end 143.47452 75.34148) (width 0.25) (layer "F.Cu") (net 17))
 (segment (start 143.47452 75.34148) (end 143.251 75.565) (width 0.25) (layer "F.Cu") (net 17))
 (segment (start 144.145 73.919) (end 144.145 72.465) (width 0.25) (layer "F.Cu") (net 13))
 (segment (start 145.791 75.565) (end 144.145 73.919) (width 0.25) (layer "F.Cu") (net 13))
 (segment (start 134.053 69.215) (end 134.053 69.918) (width 0.25) (layer "B.Cu") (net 18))
 (segment (start 134.053 69.215) (end 134.747 69.215) (width 0.25) (layer "B.Cu") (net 18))
 (segment (start 136.779 70.215) (end 135.747 70.215) (width 0.25) (layer "B.Cu") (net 18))
 (segment (start 135.747 70.215) (end 134.747 69.215) (width 0.25) (layer "B.Cu") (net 18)))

